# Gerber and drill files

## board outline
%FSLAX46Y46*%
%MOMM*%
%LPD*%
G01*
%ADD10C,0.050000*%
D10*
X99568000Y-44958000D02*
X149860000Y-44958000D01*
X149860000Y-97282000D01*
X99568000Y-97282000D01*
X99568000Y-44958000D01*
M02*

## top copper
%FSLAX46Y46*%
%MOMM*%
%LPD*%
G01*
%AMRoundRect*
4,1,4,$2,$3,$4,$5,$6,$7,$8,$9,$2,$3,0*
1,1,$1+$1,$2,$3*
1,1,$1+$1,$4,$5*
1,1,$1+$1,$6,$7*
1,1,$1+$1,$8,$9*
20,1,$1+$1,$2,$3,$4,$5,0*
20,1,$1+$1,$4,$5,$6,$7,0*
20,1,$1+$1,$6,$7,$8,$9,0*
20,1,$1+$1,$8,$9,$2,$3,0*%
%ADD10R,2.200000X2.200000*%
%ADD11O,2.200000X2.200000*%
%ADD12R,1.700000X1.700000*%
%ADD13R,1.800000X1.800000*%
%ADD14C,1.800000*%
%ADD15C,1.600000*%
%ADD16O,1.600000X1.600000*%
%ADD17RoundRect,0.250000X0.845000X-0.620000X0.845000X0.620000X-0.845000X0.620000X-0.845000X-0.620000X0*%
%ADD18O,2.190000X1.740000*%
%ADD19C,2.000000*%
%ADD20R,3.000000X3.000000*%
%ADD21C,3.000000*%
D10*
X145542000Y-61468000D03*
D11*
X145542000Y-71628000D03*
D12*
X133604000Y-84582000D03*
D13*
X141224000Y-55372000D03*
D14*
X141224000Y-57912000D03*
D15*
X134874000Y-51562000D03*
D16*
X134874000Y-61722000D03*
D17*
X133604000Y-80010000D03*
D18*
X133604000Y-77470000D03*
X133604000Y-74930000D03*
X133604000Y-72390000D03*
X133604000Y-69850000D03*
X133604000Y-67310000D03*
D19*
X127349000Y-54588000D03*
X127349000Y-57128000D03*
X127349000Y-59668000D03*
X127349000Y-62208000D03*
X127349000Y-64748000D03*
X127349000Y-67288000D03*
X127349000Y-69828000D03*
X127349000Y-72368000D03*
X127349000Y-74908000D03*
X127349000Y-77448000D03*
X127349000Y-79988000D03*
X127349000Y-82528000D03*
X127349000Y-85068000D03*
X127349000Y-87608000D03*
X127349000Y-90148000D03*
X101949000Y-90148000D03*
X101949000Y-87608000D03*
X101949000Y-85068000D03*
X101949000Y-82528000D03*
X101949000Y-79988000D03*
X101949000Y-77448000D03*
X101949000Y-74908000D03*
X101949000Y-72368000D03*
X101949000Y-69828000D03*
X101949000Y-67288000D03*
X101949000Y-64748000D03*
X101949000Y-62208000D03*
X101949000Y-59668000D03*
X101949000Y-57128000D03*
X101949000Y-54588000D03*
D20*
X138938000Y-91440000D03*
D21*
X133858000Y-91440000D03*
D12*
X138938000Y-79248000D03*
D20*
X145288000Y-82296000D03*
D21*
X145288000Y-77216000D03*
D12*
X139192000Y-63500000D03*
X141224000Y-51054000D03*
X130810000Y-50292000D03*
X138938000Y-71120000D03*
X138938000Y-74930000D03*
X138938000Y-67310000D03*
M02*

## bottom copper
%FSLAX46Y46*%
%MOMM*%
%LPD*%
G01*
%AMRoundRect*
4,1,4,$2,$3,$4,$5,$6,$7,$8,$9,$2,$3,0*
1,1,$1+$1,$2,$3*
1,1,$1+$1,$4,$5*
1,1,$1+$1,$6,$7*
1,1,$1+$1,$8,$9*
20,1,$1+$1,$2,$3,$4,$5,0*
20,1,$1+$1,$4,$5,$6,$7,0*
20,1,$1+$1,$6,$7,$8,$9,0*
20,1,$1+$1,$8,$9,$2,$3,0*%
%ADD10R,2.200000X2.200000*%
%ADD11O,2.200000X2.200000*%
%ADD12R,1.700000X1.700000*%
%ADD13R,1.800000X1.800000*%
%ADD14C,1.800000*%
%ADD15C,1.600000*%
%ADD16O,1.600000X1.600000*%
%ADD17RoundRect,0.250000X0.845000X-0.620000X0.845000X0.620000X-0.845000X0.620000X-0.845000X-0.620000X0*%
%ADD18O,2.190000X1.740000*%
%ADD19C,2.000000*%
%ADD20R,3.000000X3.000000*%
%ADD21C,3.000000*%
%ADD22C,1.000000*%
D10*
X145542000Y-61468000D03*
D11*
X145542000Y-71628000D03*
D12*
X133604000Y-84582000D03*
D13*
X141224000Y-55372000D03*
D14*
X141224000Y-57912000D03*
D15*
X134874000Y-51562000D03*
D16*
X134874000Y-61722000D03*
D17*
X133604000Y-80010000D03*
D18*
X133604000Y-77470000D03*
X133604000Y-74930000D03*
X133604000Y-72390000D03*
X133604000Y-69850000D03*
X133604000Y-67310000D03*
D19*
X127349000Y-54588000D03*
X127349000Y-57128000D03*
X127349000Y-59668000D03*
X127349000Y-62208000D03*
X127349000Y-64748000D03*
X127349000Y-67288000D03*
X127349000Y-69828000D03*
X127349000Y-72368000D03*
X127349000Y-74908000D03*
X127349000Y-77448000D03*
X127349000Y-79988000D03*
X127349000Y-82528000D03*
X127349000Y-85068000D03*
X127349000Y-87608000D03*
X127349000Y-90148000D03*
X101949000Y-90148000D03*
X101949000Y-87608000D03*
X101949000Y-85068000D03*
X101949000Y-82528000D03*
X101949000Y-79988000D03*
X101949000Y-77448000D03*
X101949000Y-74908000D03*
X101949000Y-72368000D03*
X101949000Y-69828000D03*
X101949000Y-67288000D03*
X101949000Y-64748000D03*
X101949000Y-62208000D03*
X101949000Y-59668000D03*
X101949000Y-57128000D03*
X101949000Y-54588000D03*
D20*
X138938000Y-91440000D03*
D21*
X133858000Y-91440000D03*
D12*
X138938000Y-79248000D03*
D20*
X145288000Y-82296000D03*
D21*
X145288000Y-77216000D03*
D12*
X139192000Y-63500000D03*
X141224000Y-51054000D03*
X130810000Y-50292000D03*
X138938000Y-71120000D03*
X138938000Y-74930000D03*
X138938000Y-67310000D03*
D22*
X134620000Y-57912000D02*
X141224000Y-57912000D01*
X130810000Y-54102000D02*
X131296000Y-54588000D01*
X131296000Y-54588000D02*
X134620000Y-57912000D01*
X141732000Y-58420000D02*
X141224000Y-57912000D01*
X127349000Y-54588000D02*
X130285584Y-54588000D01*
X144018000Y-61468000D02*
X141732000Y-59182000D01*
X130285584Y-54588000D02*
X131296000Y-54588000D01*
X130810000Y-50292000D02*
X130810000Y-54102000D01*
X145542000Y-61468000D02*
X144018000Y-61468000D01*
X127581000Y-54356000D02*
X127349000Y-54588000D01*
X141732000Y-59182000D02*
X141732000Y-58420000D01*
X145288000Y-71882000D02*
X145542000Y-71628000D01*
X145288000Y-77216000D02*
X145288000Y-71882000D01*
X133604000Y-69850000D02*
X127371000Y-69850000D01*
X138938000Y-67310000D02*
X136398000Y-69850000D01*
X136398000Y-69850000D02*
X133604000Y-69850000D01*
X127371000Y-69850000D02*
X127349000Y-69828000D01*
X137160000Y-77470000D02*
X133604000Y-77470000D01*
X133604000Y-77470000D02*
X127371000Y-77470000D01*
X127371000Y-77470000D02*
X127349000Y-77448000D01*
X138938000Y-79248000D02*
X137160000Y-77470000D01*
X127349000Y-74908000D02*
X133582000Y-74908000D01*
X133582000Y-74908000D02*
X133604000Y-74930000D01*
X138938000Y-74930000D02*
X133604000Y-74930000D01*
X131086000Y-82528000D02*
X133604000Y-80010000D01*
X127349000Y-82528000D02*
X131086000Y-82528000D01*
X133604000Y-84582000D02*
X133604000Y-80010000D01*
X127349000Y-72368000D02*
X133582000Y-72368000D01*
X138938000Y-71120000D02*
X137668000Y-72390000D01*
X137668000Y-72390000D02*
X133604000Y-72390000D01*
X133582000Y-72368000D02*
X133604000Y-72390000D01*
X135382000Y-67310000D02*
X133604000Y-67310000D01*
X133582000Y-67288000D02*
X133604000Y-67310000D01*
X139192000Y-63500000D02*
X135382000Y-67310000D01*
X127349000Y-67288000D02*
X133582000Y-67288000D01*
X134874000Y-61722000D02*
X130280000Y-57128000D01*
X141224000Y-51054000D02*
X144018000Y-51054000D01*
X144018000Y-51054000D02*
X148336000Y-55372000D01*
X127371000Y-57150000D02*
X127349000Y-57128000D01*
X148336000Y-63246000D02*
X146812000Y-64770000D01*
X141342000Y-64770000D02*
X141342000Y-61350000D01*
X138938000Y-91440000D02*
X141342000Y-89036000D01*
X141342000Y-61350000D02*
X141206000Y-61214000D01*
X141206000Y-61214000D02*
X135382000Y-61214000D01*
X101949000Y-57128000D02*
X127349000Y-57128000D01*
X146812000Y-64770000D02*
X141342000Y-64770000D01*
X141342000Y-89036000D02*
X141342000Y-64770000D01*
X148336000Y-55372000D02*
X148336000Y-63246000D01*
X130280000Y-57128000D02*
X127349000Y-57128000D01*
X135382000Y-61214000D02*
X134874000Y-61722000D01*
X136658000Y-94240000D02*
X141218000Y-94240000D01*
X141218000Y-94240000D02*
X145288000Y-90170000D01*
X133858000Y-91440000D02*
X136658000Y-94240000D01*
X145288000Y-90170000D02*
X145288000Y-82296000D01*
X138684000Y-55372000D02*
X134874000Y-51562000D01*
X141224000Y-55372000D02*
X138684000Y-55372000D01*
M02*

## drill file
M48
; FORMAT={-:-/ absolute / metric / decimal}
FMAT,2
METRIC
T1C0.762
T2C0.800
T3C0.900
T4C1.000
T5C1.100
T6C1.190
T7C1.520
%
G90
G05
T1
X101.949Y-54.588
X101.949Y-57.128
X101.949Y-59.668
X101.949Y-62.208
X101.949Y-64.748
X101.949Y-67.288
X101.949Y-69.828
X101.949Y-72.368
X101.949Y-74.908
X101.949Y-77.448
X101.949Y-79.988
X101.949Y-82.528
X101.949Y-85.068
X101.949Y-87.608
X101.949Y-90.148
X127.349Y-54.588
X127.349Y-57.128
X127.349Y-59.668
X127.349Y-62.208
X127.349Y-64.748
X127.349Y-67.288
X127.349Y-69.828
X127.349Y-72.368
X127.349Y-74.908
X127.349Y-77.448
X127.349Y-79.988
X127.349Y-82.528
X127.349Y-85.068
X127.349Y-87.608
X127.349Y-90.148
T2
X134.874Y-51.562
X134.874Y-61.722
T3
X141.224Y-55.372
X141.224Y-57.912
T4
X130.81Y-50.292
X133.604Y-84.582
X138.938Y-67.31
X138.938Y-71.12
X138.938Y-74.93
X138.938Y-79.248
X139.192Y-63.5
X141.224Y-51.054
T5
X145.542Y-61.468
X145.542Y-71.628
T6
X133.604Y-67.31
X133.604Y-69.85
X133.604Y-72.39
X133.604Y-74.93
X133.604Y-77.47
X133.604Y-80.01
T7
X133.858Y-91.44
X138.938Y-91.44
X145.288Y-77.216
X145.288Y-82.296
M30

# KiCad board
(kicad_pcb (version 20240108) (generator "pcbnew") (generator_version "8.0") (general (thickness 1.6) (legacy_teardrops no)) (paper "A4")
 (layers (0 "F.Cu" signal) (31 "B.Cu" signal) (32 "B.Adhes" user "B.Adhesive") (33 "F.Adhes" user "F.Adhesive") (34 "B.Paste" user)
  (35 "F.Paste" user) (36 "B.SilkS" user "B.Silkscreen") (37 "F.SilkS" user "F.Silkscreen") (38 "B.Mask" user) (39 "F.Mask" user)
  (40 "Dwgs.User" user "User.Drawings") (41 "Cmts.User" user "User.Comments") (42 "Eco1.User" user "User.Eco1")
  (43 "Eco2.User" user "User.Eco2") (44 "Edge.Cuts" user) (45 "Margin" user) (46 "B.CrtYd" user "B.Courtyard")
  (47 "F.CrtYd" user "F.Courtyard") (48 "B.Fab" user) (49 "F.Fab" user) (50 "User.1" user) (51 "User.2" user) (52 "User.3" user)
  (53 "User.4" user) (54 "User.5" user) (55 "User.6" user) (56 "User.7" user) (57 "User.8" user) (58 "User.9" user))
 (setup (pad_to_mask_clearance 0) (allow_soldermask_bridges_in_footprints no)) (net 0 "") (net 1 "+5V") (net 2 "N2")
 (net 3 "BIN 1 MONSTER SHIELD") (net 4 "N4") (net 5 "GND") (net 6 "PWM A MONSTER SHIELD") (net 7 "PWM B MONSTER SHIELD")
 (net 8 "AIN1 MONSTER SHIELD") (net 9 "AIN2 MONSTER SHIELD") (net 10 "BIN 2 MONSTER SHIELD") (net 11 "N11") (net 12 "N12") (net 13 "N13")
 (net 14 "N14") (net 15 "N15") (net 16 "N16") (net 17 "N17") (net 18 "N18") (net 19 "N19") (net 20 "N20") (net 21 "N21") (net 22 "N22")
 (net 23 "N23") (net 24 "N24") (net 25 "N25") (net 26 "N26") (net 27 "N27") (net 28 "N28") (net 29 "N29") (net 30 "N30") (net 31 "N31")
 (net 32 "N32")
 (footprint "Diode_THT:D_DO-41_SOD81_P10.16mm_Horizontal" (layer "F.Cu") (at 145.542 61.468 -90)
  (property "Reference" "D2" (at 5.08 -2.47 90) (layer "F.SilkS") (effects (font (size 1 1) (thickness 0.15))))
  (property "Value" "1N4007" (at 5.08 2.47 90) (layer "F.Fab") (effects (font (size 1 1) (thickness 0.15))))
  (pad "1" thru_hole rect (at 0 0 270) (size 2.2 2.2) (drill 1.1) (layers "*.Cu" "*.Mask") (remove_unused_layers no) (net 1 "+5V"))
  (pad "2" thru_hole oval (at 10.16 0 270) (size 2.2 2.2) (drill 1.1) (layers "*.Cu" "*.Mask") (remove_unused_layers no) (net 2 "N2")))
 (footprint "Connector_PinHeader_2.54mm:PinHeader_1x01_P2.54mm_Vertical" (layer "F.Cu") (at 133.604 84.582 90)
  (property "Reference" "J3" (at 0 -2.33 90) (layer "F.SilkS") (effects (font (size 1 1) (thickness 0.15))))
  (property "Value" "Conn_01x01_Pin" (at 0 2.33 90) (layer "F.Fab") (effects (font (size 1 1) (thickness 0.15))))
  (pad "1" thru_hole rect (at 0 0 90) (size 1.7 1.7) (drill 1) (layers "*.Cu" "*.Mask") (remove_unused_layers no)
   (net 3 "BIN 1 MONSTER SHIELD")))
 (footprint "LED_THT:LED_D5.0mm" (layer "F.Cu") (at 141.224 55.372 -90)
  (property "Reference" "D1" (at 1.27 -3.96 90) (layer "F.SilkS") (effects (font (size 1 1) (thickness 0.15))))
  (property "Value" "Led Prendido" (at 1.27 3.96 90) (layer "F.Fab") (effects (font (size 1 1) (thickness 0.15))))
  (pad "1" thru_hole rect (at 0 0 270) (size 1.8 1.8) (drill 0.9) (layers "*.Cu" "*.Mask") (remove_unused_layers no) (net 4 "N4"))
  (pad "2" thru_hole circle (at 2.54 0 270) (size 1.8 1.8) (drill 0.9) (layers "*.Cu" "*.Mask") (remove_unused_layers no) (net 1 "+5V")))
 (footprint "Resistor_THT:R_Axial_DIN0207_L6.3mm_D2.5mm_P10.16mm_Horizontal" (layer "F.Cu") (at 134.874 51.562 -90)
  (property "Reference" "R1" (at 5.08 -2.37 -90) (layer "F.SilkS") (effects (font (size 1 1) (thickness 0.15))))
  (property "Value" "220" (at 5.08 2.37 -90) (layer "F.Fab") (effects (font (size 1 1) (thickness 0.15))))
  (pad "1" thru_hole circle (at 0 0 270) (size 1.6 1.6) (drill 0.8) (layers "*.Cu" "*.Mask") (remove_unused_layers no) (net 4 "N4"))
  (pad "2" thru_hole oval (at 10.16 0 270) (size 1.6 1.6) (drill 0.8) (layers "*.Cu" "*.Mask") (remove_unused_layers no) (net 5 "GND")))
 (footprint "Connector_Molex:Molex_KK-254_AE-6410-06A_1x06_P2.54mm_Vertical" (layer "F.Cu") (at 133.604 80.01 90)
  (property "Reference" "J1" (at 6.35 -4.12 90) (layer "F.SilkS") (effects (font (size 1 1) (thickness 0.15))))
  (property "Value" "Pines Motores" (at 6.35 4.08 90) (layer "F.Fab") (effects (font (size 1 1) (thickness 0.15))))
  (pad "1" thru_hole roundrect (at 0 0 90) (size 1.74 2.19) (drill 1.19) (layers "*.Cu" "*.Mask") (remove_unused_layers no)
   (roundrect_rratio 0.143678) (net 3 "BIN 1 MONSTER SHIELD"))
  (pad "2" thru_hole oval (at 2.54 0 90) (size 1.74 2.19) (drill 1.19) (layers "*.Cu" "*.Mask") (remove_unused_layers no)
   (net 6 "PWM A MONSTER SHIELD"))
  (pad "3" thru_hole oval (at 5.08 0 90) (size 1.74 2.19) (drill 1.19) (layers "*.Cu" "*.Mask") (remove_unused_layers no)
   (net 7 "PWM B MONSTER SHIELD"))
  (pad "4" thru_hole oval (at 7.62 0 90) (size 1.74 2.19) (drill 1.19) (layers "*.Cu" "*.Mask") (remove_unused_layers no)
   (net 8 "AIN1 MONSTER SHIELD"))
  (pad "5" thru_hole oval (at 10.16 0 90) (size 1.74 2.19) (drill 1.19) (layers "*.Cu" "*.Mask") (remove_unused_layers no)
   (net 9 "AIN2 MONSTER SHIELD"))
  (pad "6" thru_hole oval (at 12.7 0 90) (size 1.74 2.19) (drill 1.19) (layers "*.Cu" "*.Mask") (remove_unused_layers no)
   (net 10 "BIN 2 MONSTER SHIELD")))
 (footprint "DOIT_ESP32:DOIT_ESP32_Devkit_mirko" (layer "F.Cu") (at 100.679 45.698)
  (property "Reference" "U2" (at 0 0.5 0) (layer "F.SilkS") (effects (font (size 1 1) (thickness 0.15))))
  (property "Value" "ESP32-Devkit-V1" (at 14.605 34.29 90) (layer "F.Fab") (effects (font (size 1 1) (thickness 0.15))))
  (pad "1" thru_hole circle (at 26.67 8.89) (size 2 2) (drill 0.762) (layers "*.Cu" "*.Mask") (remove_unused_layers no) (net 1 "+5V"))
  (pad "2" thru_hole circle (at 26.67 11.43) (size 2 2) (drill 0.762) (layers "*.Cu" "*.Mask") (remove_unused_layers no) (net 5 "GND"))
  (pad "3" thru_hole circle (at 26.67 13.97) (size 2 2) (drill 0.762) (layers "*.Cu" "*.Mask") (remove_unused_layers no) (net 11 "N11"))
  (pad "4" thru_hole circle (at 26.67 16.51) (size 2 2) (drill 0.762) (layers "*.Cu" "*.Mask") (remove_unused_layers no) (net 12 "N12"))
  (pad "5" thru_hole circle (at 26.67 19.05) (size 2 2) (drill 0.762) (layers "*.Cu" "*.Mask") (remove_unused_layers no) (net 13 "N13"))
  (pad "6" thru_hole circle (at 26.67 21.59) (size 2 2) (drill 0.762) (layers "*.Cu" "*.Mask") (remove_unused_layers no)
   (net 10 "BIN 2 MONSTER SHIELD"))
  (pad "7" thru_hole circle (at 26.67 24.13) (size 2 2) (drill 0.762) (layers "*.Cu" "*.Mask") (remove_unused_layers no)
   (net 9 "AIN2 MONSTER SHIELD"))
  (pad "8" thru_hole circle (at 26.67 26.67) (size 2 2) (drill 0.762) (layers "*.Cu" "*.Mask") (remove_unused_layers no)
   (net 8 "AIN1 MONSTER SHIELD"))
  (pad "9" thru_hole circle (at 26.67 29.21) (size 2 2) (drill 0.762) (layers "*.Cu" "*.Mask") (remove_unused_layers no)
   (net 7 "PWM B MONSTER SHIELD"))
  (pad "10" thru_hole circle (at 26.67 31.75) (size 2 2) (drill 0.762) (layers "*.Cu" "*.Mask") (remove_unused_layers no)
   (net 6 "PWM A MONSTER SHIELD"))
  (pad "11" thru_hole circle (at 26.67 34.29) (size 2 2) (drill 0.762) (layers "*.Cu" "*.Mask") (remove_unused_layers no) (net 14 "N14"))
  (pad "12" thru_hole circle (at 26.67 36.83) (size 2 2) (drill 0.762) (layers "*.Cu" "*.Mask") (remove_unused_layers no)
   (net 3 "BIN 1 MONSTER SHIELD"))
  (pad "13" thru_hole circle (at 26.67 39.37) (size 2 2) (drill 0.762) (layers "*.Cu" "*.Mask") (remove_unused_layers no) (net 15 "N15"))
  (pad "14" thru_hole circle (at 26.67 41.91) (size 2 2) (drill 0.762) (layers "*.Cu" "*.Mask") (remove_unused_layers no) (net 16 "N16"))
  (pad "15" thru_hole circle (at 26.67 44.45) (size 2 2) (drill 0.762) (layers "*.Cu" "*.Mask") (remove_unused_layers no) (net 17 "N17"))
  (pad "16" thru_hole circle (at 1.27 44.45) (size 2 2) (drill 0.762) (layers "*.Cu" "*.Mask") (remove_unused_layers no) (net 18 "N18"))
  (pad "17" thru_hole circle (at 1.27 41.91) (size 2 2) (drill 0.762) (layers "*.Cu" "*.Mask") (remove_unused_layers no) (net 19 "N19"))
  (pad "18" thru_hole circle (at 1.27 39.37) (size 2 2) (drill 0.762) (layers "*.Cu" "*.Mask") (remove_unused_layers no) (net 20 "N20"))
  (pad "19" thru_hole circle (at 1.27 36.83) (size 2 2) (drill 0.762) (layers "*.Cu" "*.Mask") (remove_unused_layers no) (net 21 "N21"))
  (pad "20" thru_hole circle (at 1.27 34.29) (size 2 2) (drill 0.762) (layers "*.Cu" "*.Mask") (remove_unused_layers no) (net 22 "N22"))
  (pad "21" thru_hole circle (at 1.27 31.75) (size 2 2) (drill 0.762) (layers "*.Cu" "*.Mask") (remove_unused_layers no) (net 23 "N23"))
  (pad "22" thru_hole circle (at 1.27 29.21) (size 2 2) (drill 0.762) (layers "*.Cu" "*.Mask") (remove_unused_layers no) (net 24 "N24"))
  (pad "23" thru_hole circle (at 1.27 26.67) (size 2 2) (drill 0.762) (layers "*.Cu" "*.Mask") (remove_unused_layers no) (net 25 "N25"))
  (pad "24" thru_hole circle (at 1.27 24.13) (size 2 2) (drill 0.762) (layers "*.Cu" "*.Mask") (remove_unused_layers no) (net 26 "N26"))
  (pad "25" thru_hole circle (at 1.27 21.59) (size 2 2) (drill 0.762) (layers "*.Cu" "*.Mask") (remove_unused_layers no) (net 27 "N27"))
  (pad "26" thru_hole circle (at 1.27 19.05) (size 2 2) (drill 0.762) (layers "*.Cu" "*.Mask") (remove_unused_layers no) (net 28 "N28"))
  (pad "27" thru_hole circle (at 1.27 16.51) (size 2 2) (drill 0.762) (layers "*.Cu" "*.Mask") (remove_unused_layers no) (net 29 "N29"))
  (pad "28" thru_hole circle (at 1.27 13.97) (size 2 2) (drill 0.762) (layers "*.Cu" "*.Mask") (remove_unused_layers no) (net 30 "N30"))
  (pad "29" thru_hole circle (at 1.27 11.43) (size 2 2) (drill 0.762) (layers "*.Cu" "*.Mask") (remove_unused_layers no) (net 5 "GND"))
  (pad "30" thru_hole circle (at 1.27 8.89) (size 2 2) (drill 0.762) (layers "*.Cu" "*.Mask") (remove_unused_layers no) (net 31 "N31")))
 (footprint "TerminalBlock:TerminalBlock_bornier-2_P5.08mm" (layer "F.Cu") (at 138.938 91.44 180)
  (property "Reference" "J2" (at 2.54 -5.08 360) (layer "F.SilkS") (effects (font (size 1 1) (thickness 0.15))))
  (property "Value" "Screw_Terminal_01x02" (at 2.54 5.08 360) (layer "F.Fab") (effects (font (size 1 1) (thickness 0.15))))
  (pad "1" thru_hole rect (at 0 0 180) (size 3 3) (drill 1.52) (layers "*.Cu" "*.Mask") (remove_unused_layers no) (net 5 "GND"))
  (pad "2" thru_hole circle (at 5.08 0 180) (size 3 3) (drill 1.52) (layers "*.Cu" "*.Mask") (remove_unused_layers no) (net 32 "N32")))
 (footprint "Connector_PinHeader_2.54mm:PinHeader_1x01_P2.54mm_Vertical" (layer "F.Cu") (at 138.938 79.248 90)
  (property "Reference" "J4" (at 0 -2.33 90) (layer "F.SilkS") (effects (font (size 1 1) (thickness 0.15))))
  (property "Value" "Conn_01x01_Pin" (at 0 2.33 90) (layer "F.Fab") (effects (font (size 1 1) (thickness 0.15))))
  (pad "1" thru_hole rect (at 0 0 90) (size 1.7 1.7) (drill 1) (layers "*.Cu" "*.Mask") (remove_unused_layers no)
   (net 6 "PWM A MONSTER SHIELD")))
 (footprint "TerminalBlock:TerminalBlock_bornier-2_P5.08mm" (layer "F.Cu") (at 145.288 82.296 90)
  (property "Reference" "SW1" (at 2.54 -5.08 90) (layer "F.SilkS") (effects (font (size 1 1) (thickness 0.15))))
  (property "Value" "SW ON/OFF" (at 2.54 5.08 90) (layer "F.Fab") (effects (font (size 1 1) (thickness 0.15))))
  (pad "1" thru_hole rect (at 0 0 90) (size 3 3) (drill 1.52) (layers "*.Cu" "*.Mask") (remove_unused_layers no) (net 32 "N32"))
  (pad "2" thru_hole circle (at 5.08 0 90) (size 3 3) (drill 1.52) (layers "*.Cu" "*.Mask") (remove_unused_layers no) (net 2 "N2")))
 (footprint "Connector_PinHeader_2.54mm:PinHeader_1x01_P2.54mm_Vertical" (layer "F.Cu") (at 139.192 63.5 90)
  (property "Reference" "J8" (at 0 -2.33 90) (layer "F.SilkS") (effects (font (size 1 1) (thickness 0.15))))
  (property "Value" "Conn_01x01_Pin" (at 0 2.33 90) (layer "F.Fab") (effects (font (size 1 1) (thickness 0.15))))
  (pad "1" thru_hole rect (at 0 0 90) (size 1.7 1.7) (drill 1) (layers "*.Cu" "*.Mask") (remove_unused_layers no)
   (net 10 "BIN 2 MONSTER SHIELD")))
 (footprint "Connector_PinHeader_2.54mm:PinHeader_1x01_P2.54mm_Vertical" (layer "F.Cu") (at 141.224 51.054 90)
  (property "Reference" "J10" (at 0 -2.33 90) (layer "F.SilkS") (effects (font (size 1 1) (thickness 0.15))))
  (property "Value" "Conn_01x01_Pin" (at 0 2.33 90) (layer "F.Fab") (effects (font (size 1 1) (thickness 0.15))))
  (pad "1" thru_hole rect (at 0 0 90) (size 1.7 1.7) (drill 1) (layers "*.Cu" "*.Mask") (remove_unused_layers no) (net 5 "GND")))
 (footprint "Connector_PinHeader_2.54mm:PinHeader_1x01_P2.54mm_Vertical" (layer "F.Cu") (at 130.81 50.292 90)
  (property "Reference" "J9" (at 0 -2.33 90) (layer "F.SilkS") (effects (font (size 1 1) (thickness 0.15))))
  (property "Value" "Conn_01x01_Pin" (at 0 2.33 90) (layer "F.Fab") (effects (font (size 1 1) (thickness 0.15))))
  (pad "1" thru_hole rect (at 0 0 90) (size 1.7 1.7) (drill 1) (layers "*.Cu" "*.Mask") (remove_unused_layers no) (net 1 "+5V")))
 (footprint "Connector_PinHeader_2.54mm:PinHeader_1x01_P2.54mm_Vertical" (layer "F.Cu") (at 138.938 71.12 90)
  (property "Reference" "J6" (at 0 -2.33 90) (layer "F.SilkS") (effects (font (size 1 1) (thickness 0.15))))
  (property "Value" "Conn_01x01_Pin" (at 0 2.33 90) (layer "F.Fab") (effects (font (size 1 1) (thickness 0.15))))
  (pad "1" thru_hole rect (at 0 0 90) (size 1.7 1.7) (drill 1) (layers "*.Cu" "*.Mask") (remove_unused_layers no)
   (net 8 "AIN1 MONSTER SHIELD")))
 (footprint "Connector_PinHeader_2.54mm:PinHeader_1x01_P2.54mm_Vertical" (layer "F.Cu") (at 138.938 74.93 90)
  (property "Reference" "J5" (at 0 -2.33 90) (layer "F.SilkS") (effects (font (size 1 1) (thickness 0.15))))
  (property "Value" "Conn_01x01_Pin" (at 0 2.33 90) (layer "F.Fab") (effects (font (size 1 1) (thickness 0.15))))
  (pad "1" thru_hole rect (at 0 0 90) (size 1.7 1.7) (drill 1) (layers "*.Cu" "*.Mask") (remove_unused_layers no)
   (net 7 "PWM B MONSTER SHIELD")))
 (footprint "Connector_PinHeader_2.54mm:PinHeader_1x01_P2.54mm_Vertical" (layer "F.Cu") (at 138.938 67.31 90)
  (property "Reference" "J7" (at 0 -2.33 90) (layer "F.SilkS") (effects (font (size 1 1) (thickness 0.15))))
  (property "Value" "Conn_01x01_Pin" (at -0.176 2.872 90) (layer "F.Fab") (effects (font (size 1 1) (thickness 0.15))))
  (pad "1" thru_hole rect (at 0 0 90) (size 1.7 1.7) (drill 1) (layers "*.Cu" "*.Mask") (remove_unused_layers no)
   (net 9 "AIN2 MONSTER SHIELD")))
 (gr_rect (start 99.568 44.958) (end 149.86 97.282) (stroke (width 0.05) (type default)) (fill none) (layer "Edge.Cuts"))
 (segment (start 134.62 57.912) (end 141.224 57.912) (width 1) (layer "B.Cu") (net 1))
 (segment (start 130.81 54.102) (end 131.296 54.588) (width 1) (layer "B.Cu") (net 1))
 (segment (start 131.296 54.588) (end 134.62 57.912) (width 1) (layer "B.Cu") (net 1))
 (segment (start 141.732 58.42) (end 141.224 57.912) (width 1) (layer "B.Cu") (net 1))
 (segment (start 127.349 54.588) (end 130.285584 54.588) (width 1) (layer "B.Cu") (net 1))
 (segment (start 144.018 61.468) (end 141.732 59.182) (width 1) (layer "B.Cu") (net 1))
 (segment (start 130.285584 54.588) (end 131.296 54.588) (width 1) (layer "B.Cu") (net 1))
 (segment (start 130.81 50.292) (end 130.81 54.102) (width 1) (layer "B.Cu") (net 1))
 (segment (start 145.542 61.468) (end 144.018 61.468) (width 1) (layer "B.Cu") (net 1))
 (segment (start 127.581 54.356) (end 127.349 54.588) (width 1) (layer "B.Cu") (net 1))
 (segment (start 141.732 59.182) (end 141.732 58.42) (width 1) (layer "B.Cu") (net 1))
 (segment (start 145.288 71.882) (end 145.542 71.628) (width 1) (layer "B.Cu") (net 2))
 (segment (start 145.288 77.216) (end 145.288 71.882) (width 1) (layer "B.Cu") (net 2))
 (segment (start 133.604 69.85) (end 127.371 69.85) (width 1) (layer "B.Cu") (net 9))
 (segment (start 138.938 67.31) (end 136.398 69.85) (width 1) (layer "B.Cu") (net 9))
 (segment (start 136.398 69.85) (end 133.604 69.85) (width 1) (layer "B.Cu") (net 9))
 (segment (start 127.371 69.85) (end 127.349 69.828) (width 1) (layer "B.Cu") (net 9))
 (segment (start 137.16 77.47) (end 133.604 77.47) (width 1) (layer "B.Cu") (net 6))
 (segment (start 133.604 77.47) (end 127.371 77.47) (width 1) (layer "B.Cu") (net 6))
 (segment (start 127.371 77.47) (end 127.349 77.448) (width 1) (layer "B.Cu") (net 6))
 (segment (start 138.938 79.248) (end 137.16 77.47) (width 1) (layer "B.Cu") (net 6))
 (segment (start 127.349 74.908) (end 133.582 74.908) (width 1) (layer "B.Cu") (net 7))
 (segment (start 133.582 74.908) (end 133.604 74.93) (width 1) (layer "B.Cu") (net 7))
 (segment (start 138.938 74.93) (end 133.604 74.93) (width 1) (layer "B.Cu") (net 7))
 (segment (start 131.086 82.528) (end 133.604 80.01) (width 1) (layer "B.Cu") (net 3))
 (segment (start 127.349 82.528) (end 131.086 82.528) (width 1) (layer "B.Cu") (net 3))
 (segment (start 133.604 84.582) (end 133.604 80.01) (width 1) (layer "B.Cu") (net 3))
 (segment (start 127.349 72.368) (end 133.582 72.368) (width 1) (layer "B.Cu") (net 8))
 (segment (start 138.938 71.12) (end 137.668 72.39) (width 1) (layer "B.Cu") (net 8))
 (segment (start 137.668 72.39) (end 133.604 72.39) (width 1) (layer "B.Cu") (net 8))
 (segment (start 133.582 72.368) (end 133.604 72.39) (width 1) (layer "B.Cu") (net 8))
 (segment (start 135.382 67.31) (end 133.604 67.31) (width 1) (layer "B.Cu") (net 10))
 (segment (start 133.582 67.288) (end 133.604 67.31) (width 1) (layer "B.Cu") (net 10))
 (segment (start 139.192 63.5) (end 135.382 67.31) (width 1) (layer "B.Cu") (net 10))
 (segment (start 127.349 67.288) (end 133.582 67.288) (width 1) (layer "B.Cu") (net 10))
 (segment (start 134.874 61.722) (end 130.28 57.128) (width 1) (layer "B.Cu") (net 5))
 (segment (start 141.224 51.054) (end 144.018 51.054) (width 1) (layer "B.Cu") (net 5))
 (segment (start 144.018 51.054) (end 148.336 55.372) (width 1) (layer "B.Cu") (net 5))
 (segment (start 127.371 57.15) (end 127.349 57.128) (width 1) (layer "B.Cu") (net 5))
 (segment (start 148.336 63.246) (end 146.812 64.77) (width 1) (layer "B.Cu") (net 5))
 (segment (start 141.342 64.77) (end 141.342 61.35) (width 1) (layer "B.Cu") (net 5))
 (segment (start 138.938 91.44) (end 141.342 89.036) (width 1) (layer "B.Cu") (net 5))
 (segment (start 141.342 61.35) (end 141.206 61.214) (width 1) (layer "B.Cu") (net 5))
 (segment (start 141.206 61.214) (end 135.382 61.214) (width 1) (layer "B.Cu") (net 5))
 (segment (start 101.949 57.128) (end 127.349 57.128) (width 1) (layer "B.Cu") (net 5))
 (segment (start 146.812 64.77) (end 141.342 64.77) (width 1) (layer "B.Cu") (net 5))
 (segment (start 141.342 89.036) (end 141.342 64.77) (width 1) (layer "B.Cu") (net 5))
 (segment (start 148.336 55.372) (end 148.336 63.246) (width 1) (layer "B.Cu") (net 5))
 (segment (start 130.28 57.128) (end 127.349 57.128) (width 1) (layer "B.Cu") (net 5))
 (segment (start 135.382 61.214) (end 134.874 61.722) (width 1) (layer "B.Cu") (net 5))
 (segment (start 136.658 94.24) (end 141.218 94.24) (width 1) (layer "B.Cu") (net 32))
 (segment (start 141.218 94.24) (end 145.288 90.17) (width 1) (layer "B.Cu") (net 32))
 (segment (start 133.858 91.44) (end 136.658 94.24) (width 1) (layer "B.Cu") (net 32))
 (segment (start 145.288 90.17) (end 145.288 82.296) (width 1) (layer "B.Cu") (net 32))
 (segment (start 138.684 55.372) (end 134.874 51.562) (width 1) (layer "B.Cu") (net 4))
 (segment (start 141.224 55.372) (end 138.684 55.372) (width 1) (layer "B.Cu") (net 4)))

